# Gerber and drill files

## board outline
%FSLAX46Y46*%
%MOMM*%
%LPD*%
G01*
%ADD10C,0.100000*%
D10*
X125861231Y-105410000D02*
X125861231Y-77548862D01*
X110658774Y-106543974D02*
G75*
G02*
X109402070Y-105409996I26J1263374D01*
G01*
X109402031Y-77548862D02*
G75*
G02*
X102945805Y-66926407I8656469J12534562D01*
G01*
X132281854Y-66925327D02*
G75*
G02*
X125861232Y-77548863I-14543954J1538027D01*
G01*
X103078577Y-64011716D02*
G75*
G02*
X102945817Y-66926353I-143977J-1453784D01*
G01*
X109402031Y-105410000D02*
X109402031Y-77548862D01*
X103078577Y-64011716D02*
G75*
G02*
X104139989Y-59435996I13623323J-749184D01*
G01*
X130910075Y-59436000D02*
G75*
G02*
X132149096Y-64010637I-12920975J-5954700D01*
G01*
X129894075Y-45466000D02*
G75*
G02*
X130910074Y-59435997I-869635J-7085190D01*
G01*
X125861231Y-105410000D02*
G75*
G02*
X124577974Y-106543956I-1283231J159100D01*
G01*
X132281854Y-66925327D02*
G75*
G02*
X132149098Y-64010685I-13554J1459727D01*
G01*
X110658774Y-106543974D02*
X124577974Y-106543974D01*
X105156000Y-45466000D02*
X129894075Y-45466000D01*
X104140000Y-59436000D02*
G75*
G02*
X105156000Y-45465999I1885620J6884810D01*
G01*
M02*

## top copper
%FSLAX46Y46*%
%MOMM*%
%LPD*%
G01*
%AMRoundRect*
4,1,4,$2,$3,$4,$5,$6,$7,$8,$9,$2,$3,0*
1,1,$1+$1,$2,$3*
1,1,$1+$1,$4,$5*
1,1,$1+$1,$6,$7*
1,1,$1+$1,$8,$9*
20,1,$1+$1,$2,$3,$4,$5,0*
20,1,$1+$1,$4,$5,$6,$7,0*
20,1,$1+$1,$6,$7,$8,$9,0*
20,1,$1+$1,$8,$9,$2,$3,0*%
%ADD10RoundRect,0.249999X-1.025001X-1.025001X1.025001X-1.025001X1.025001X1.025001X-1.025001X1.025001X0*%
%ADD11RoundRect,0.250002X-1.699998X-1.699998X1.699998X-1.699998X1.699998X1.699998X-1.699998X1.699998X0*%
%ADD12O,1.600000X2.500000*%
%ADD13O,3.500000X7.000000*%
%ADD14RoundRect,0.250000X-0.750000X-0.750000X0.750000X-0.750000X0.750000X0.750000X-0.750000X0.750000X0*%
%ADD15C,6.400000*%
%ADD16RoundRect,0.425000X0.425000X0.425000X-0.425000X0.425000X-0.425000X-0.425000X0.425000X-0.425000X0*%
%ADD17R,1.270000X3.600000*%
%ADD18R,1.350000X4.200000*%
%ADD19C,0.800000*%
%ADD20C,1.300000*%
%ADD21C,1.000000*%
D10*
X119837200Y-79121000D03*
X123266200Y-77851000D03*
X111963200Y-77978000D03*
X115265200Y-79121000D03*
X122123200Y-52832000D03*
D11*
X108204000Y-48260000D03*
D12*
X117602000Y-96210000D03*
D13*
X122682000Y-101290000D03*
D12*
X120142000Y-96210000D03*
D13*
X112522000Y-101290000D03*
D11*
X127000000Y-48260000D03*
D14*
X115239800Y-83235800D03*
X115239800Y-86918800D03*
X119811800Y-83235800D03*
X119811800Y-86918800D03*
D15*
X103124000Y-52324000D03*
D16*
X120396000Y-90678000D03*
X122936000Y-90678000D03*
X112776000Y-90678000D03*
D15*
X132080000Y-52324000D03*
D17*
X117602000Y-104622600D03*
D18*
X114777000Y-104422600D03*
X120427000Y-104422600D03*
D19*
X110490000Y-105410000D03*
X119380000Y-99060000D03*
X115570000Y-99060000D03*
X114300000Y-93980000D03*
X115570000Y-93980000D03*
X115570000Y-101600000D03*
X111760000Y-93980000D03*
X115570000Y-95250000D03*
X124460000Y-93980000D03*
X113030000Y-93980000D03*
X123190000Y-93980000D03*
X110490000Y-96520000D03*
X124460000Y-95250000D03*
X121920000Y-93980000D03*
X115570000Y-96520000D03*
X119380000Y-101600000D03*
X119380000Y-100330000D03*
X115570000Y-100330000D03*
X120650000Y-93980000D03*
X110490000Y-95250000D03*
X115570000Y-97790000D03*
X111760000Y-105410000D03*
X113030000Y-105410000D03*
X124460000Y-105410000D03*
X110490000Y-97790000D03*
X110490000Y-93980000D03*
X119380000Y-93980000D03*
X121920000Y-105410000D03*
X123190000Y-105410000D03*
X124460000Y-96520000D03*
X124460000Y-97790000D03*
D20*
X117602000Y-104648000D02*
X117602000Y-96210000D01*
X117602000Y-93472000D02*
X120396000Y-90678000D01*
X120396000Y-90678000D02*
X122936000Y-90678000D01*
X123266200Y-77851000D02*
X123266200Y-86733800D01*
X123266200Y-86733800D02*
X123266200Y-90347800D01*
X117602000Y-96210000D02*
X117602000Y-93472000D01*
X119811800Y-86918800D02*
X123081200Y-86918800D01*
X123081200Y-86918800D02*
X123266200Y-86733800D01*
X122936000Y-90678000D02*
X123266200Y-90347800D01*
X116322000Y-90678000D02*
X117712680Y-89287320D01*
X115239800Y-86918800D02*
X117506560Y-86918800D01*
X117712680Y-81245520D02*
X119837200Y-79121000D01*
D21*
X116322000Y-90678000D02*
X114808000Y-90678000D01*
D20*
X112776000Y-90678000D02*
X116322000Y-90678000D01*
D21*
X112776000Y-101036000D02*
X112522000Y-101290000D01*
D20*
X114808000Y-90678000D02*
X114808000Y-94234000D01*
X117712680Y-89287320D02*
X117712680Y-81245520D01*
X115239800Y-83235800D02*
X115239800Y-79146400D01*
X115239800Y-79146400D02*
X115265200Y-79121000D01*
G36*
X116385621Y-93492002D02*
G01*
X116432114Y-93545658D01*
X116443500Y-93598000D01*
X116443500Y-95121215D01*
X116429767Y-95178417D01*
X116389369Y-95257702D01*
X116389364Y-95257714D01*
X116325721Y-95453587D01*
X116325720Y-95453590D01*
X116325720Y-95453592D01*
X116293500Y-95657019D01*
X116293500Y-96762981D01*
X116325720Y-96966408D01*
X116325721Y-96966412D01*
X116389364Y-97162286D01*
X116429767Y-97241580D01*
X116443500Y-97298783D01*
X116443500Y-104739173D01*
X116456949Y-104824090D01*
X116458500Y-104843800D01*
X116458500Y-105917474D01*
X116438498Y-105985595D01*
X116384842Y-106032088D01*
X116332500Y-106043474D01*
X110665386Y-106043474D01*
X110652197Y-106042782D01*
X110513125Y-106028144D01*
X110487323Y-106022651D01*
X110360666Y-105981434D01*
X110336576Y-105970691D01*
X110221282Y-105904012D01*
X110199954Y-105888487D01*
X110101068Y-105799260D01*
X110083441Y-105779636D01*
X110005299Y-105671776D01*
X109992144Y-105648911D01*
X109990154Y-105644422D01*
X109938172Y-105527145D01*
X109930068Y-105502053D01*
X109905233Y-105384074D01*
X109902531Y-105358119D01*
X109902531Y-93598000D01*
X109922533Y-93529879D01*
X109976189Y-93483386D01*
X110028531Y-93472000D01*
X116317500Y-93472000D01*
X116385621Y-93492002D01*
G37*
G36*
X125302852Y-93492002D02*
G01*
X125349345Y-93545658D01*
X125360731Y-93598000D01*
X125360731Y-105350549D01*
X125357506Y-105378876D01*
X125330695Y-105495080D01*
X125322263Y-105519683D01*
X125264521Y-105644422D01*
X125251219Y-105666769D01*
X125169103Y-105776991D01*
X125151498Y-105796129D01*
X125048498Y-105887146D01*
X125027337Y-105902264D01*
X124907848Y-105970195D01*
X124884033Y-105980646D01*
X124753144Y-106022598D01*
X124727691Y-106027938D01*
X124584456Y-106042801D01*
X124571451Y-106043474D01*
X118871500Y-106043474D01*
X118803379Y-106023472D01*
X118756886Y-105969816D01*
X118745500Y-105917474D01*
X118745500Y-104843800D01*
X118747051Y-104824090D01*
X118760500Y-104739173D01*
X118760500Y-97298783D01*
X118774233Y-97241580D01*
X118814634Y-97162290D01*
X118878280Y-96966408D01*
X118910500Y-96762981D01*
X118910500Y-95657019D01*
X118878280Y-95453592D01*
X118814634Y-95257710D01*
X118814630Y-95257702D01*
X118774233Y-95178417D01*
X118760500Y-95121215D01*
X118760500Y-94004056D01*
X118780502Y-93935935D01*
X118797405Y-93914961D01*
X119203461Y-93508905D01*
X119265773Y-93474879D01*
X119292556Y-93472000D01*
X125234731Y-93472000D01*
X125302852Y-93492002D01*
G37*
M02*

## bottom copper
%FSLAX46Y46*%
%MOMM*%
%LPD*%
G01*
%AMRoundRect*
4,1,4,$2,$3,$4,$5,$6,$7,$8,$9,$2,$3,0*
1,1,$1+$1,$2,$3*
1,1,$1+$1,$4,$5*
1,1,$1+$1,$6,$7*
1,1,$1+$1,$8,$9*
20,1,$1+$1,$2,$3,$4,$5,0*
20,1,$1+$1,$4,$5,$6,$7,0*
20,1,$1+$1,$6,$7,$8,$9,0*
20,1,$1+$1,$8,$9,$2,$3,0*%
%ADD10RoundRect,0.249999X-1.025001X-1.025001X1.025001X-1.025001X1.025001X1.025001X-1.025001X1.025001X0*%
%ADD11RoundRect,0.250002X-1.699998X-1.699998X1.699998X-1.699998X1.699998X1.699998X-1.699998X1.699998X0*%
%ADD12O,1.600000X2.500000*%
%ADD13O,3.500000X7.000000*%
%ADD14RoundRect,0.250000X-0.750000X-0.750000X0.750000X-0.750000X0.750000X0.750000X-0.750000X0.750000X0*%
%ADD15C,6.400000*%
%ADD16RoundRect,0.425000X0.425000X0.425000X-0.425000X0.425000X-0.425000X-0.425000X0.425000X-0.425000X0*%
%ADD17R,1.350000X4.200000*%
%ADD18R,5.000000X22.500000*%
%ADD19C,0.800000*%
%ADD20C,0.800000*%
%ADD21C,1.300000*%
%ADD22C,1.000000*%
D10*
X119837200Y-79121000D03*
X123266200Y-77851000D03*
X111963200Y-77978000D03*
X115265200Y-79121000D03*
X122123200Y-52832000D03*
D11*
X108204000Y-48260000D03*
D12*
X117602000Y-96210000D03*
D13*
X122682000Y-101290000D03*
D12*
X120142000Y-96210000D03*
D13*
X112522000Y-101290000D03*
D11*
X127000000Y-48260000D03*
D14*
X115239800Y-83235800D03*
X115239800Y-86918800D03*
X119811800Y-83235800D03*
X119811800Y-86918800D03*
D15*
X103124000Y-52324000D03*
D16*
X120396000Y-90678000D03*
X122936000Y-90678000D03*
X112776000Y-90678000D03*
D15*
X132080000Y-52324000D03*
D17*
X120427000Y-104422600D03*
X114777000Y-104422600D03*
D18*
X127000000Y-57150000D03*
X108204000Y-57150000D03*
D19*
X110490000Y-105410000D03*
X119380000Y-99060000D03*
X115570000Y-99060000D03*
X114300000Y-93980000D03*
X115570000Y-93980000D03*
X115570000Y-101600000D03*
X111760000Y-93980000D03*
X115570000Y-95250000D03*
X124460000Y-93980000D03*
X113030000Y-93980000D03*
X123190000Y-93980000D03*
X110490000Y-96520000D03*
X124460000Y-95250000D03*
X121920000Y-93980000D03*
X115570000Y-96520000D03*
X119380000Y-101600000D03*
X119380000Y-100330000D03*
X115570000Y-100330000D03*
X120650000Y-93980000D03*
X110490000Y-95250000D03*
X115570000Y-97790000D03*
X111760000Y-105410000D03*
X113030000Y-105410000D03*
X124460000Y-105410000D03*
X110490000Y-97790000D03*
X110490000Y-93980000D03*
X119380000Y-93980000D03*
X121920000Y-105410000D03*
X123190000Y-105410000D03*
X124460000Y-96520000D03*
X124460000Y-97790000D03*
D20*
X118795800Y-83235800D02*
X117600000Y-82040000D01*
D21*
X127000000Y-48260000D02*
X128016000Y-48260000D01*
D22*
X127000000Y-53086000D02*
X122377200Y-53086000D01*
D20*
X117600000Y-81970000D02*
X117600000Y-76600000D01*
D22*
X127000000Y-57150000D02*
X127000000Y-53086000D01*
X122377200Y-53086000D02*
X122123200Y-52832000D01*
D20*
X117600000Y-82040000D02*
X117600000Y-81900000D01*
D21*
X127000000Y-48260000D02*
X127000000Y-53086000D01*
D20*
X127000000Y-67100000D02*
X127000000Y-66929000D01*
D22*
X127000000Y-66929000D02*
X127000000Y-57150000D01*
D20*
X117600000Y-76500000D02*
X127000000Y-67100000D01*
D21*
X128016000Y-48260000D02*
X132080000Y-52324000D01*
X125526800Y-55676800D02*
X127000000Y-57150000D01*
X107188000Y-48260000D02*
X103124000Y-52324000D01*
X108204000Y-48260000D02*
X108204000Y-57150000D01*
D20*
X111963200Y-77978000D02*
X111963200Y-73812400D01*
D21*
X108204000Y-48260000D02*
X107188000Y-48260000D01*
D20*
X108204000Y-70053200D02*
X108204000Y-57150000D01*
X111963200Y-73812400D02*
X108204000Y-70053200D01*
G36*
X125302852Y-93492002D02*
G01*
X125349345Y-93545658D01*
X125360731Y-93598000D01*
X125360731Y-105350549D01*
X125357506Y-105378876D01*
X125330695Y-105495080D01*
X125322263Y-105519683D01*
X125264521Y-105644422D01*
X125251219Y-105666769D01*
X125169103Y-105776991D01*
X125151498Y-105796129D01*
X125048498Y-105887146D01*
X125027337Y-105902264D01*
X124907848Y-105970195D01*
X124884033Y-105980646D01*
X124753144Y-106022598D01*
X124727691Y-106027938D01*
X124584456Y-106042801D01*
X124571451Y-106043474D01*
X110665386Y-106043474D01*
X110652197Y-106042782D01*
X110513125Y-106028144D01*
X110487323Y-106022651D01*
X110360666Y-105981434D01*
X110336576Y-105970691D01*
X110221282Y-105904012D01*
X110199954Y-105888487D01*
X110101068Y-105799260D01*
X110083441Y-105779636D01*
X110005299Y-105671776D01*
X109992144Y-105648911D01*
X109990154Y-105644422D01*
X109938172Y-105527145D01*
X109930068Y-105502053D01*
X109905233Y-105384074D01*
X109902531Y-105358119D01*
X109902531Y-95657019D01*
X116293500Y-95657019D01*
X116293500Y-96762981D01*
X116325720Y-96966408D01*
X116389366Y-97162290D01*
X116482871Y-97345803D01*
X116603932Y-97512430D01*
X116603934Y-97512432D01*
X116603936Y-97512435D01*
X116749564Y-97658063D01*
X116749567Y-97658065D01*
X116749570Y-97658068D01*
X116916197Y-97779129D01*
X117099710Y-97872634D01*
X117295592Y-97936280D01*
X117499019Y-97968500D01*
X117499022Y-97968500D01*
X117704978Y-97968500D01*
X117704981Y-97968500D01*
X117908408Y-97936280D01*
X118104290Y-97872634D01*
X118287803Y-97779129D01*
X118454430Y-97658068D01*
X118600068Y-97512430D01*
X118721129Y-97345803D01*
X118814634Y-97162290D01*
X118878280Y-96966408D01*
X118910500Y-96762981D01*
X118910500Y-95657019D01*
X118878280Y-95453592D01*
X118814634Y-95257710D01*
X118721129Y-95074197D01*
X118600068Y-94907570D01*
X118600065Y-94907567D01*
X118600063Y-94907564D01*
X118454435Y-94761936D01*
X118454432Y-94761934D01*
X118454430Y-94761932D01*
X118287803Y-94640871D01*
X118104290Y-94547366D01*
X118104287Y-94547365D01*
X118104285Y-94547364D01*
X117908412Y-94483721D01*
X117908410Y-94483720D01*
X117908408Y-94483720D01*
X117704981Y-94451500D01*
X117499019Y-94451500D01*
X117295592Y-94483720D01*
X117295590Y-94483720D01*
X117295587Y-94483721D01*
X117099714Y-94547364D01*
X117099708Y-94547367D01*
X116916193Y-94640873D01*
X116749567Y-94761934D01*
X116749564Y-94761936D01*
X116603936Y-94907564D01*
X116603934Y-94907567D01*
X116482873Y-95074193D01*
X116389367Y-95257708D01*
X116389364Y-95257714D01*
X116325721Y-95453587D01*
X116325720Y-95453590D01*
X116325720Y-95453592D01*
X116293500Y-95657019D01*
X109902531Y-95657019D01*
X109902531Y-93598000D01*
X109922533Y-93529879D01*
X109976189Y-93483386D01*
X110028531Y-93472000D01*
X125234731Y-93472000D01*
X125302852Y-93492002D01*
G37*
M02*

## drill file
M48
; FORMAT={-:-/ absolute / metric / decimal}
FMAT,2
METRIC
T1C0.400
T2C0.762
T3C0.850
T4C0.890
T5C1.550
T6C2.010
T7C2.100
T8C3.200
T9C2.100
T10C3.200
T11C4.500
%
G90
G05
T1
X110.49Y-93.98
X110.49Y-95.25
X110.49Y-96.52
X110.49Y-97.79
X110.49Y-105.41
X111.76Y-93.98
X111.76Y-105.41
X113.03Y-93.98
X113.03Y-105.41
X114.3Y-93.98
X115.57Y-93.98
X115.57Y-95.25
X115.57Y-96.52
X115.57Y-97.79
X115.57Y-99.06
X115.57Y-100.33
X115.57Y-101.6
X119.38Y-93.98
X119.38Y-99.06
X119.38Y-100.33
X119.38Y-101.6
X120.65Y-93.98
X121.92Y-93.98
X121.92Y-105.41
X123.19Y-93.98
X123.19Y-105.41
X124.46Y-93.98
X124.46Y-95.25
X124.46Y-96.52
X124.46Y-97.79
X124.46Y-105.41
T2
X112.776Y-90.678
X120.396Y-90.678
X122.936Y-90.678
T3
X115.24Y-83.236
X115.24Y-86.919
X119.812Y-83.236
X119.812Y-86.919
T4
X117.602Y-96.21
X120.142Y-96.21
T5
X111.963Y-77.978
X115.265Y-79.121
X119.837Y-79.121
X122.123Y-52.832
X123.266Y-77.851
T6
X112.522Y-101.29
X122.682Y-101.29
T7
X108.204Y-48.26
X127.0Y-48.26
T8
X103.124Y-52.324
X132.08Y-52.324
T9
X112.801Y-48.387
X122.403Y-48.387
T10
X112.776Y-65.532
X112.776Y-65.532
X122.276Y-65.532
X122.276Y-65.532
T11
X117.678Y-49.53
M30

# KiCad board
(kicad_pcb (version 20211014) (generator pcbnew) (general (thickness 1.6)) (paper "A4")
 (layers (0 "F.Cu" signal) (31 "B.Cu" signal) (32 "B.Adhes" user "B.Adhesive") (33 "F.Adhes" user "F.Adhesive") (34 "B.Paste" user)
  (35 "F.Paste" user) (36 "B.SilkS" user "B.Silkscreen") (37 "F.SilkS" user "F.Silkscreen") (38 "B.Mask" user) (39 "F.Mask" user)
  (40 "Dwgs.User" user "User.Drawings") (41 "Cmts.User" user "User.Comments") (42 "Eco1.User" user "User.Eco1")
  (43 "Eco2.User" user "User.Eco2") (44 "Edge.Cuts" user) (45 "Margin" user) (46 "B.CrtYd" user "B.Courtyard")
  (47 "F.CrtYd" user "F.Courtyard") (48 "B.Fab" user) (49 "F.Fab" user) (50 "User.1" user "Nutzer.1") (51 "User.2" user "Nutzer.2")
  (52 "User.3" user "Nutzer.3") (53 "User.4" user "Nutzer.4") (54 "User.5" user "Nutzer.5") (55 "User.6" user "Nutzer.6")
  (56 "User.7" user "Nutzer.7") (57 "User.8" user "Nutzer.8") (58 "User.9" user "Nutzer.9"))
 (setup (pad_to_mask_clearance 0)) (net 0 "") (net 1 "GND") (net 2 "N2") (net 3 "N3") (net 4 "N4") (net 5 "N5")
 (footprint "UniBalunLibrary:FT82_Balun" (layer "F.Cu") (at 117.602 65.532)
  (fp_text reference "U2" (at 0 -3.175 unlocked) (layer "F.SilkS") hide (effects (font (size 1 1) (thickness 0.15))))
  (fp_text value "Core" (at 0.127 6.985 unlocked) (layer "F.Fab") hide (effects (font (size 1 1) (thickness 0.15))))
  (pad "" np_thru_hole circle (at 4.6736 0) (size 3.2 3.2) (drill 3.2) (layers *.Cu *.Mask))
  (pad "" np_thru_hole circle (at -4.826 0) (size 3.2 3.2) (drill 3.2) (layers *.Cu *.Mask))
  (pad "" np_thru_hole circle (at -4.826 0) (size 3.2 3.2) (drill 3.2) (layers *.Cu *.Mask))
  (pad "" np_thru_hole circle (at 4.6736 0) (size 3.2 3.2) (drill 3.2) (layers *.Cu *.Mask))
  (pad "1" thru_hole roundrect (at 2.2352 13.589) (size 2.55 2.55) (drill 1.55) (layers *.Cu *.Mask) (roundrect_rratio 0.098039)
   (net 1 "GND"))
  (pad "2" thru_hole roundrect (at 5.6642 12.319) (size 2.55 2.55) (drill 1.55) (layers *.Cu *.Mask) (roundrect_rratio 0.098039)
   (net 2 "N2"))
  (pad "3" thru_hole roundrect (at -5.6388 12.446) (size 2.55 2.55) (drill 1.55) (layers *.Cu *.Mask) (roundrect_rratio 0.098039)
   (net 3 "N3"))
  (pad "4" thru_hole roundrect (at -2.3368 13.589) (size 2.55 2.55) (drill 1.55) (layers *.Cu *.Mask) (roundrect_rratio 0.098039)
   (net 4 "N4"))
  (pad "5" thru_hole roundrect (at 4.5212 -12.7) (size 2.55 2.55) (drill 1.55) (layers *.Cu *.Mask) (roundrect_rratio 0.098039) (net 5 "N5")))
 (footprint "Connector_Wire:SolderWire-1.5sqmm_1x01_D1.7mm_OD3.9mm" (layer "F.Cu") (at 108.204 48.26)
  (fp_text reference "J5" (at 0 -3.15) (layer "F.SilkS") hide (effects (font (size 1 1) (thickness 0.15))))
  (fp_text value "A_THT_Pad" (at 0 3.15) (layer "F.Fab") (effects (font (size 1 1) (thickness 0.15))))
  (pad "1" thru_hole roundrect (at 0 0) (size 3.9 3.9) (drill 2.1) (layers *.Cu *.Mask) (roundrect_rratio 0.064103) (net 3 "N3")))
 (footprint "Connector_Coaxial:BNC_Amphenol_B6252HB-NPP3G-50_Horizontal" (layer "F.Cu") (at 117.602 96.21 180)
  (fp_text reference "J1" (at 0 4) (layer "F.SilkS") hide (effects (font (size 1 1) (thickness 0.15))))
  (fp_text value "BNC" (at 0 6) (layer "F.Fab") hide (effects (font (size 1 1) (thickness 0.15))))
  (pad "1" thru_hole oval (at 0 0 180) (size 1.6 2.5) (drill 0.89) (layers *.Cu *.Mask) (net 2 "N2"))
  (pad "2" thru_hole oval (at -5.08 -5.08 180) (size 3.5 7) (drill 2.01) (layers *.Cu *.Mask) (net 1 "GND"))
  (pad "2" thru_hole oval (at -2.54 0 180) (size 1.6 2.5) (drill 0.89) (layers *.Cu *.Mask) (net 1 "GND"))
  (pad "2" thru_hole oval (at 5.08 -5.08 180) (size 3.5 7) (drill 2.01) (layers *.Cu *.Mask) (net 1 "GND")))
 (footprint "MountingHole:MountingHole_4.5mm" (layer "F.Cu") (at 117.6782 49.53)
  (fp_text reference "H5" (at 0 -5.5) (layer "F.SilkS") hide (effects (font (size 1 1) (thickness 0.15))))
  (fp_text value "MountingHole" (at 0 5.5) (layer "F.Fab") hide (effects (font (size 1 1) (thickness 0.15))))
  (pad "" np_thru_hole circle (at 0 0) (size 4.5 4.5) (drill 4.5) (layers *.Cu *.Mask)))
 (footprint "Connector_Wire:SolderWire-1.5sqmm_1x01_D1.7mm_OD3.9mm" (layer "F.Cu") (at 127 48.26)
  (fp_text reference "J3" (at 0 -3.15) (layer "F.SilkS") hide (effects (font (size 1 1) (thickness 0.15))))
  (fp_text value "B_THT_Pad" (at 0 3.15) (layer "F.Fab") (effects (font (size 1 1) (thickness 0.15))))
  (pad "1" thru_hole roundrect (at 0 0) (size 3.9 3.9) (drill 2.1) (layers *.Cu *.Mask) (roundrect_rratio 0.064103) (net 5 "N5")))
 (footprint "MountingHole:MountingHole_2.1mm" (layer "F.Cu") (at 112.8014 48.387)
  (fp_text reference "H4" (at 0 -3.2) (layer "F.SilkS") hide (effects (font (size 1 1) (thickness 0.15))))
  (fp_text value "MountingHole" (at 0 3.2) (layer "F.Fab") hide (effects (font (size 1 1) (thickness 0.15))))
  (pad "" np_thru_hole circle (at 0 0) (size 2.1 2.1) (drill 2.1) (layers *.Cu *.Mask)))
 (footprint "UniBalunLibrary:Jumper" (layer "F.Cu") (at 117.602 85.09)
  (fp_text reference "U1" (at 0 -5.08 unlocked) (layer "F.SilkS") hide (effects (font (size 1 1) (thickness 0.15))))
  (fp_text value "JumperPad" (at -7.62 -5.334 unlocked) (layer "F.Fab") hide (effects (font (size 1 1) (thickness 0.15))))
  (pad "1" thru_hole roundrect (at -2.3622 -1.8542) (size 2 2) (drill 0.85) (layers *.Cu *.Mask) (roundrect_rratio 0.125) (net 4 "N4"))
  (pad "2" thru_hole roundrect (at -2.3622 1.8288) (size 2 2) (drill 0.85) (layers *.Cu *.Mask) (roundrect_rratio 0.125) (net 1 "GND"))
  (pad "3" thru_hole roundrect (at 2.2098 -1.8542) (size 2 2) (drill 0.85) (layers *.Cu *.Mask) (roundrect_rratio 0.125) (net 5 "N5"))
  (pad "4" thru_hole roundrect (at 2.2098 1.8288) (size 2 2) (drill 0.85) (layers *.Cu *.Mask) (roundrect_rratio 0.125) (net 2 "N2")))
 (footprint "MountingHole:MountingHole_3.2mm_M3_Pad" (layer "F.Cu") (at 103.124 52.324)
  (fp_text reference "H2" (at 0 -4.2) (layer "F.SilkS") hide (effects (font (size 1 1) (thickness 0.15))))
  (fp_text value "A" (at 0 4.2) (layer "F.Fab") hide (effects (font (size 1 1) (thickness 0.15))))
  (pad "1" thru_hole circle (at 0 0) (size 6.4 6.4) (drill 3.2) (layers *.Cu *.Mask) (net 3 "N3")))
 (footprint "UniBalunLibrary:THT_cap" (layer "F.Cu") (at 117.856 90.678 180)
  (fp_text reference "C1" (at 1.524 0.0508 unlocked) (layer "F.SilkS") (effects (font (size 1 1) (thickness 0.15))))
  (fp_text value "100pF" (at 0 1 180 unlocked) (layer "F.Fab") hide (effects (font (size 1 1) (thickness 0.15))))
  (pad "1" thru_hole roundrect (at -2.54 0 180) (size 1.7 1.7) (drill 0.762) (layers *.Cu *.Mask) (roundrect_rratio 0.25) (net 2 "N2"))
  (pad "1" thru_hole roundrect (at -5.08 0 180) (size 1.7 1.7) (drill 0.762) (layers *.Cu *.Mask) (roundrect_rratio 0.25) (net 2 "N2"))
  (pad "2" thru_hole roundrect (at 5.08 0 180) (size 1.7 1.7) (drill 0.762) (layers *.Cu *.Mask) (roundrect_rratio 0.25) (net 1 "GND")))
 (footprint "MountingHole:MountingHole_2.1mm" (layer "F.Cu") (at 122.4026 48.387)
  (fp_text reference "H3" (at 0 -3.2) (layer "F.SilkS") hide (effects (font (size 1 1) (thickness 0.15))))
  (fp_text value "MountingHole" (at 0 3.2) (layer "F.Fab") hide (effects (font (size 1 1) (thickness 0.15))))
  (pad "" np_thru_hole circle (at 0 0) (size 2.1 2.1) (drill 2.1) (layers *.Cu *.Mask)))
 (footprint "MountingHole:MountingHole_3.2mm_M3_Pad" (layer "F.Cu") (at 132.08 52.324)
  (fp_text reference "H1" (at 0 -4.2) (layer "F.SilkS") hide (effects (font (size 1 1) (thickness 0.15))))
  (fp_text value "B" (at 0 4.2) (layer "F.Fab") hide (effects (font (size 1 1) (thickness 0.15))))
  (pad "1" thru_hole circle (at 0 0) (size 6.4 6.4) (drill 3.2) (layers *.Cu *.Mask) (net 5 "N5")))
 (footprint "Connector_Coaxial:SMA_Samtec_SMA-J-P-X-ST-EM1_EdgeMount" (layer "F.Cu") (at 117.602 104.4226)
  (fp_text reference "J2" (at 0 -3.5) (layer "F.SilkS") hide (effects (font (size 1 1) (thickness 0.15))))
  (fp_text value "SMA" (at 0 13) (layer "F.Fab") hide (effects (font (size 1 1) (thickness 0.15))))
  (pad "1" smd rect (at 0 0.2) (size 1.27 3.6) (layers "F.Cu" "F.Paste" "F.Mask") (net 2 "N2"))
  (pad "2" smd rect (at 2.825 0) (size 1.35 4.2) (layers "B.Cu" "B.Paste" "B.Mask") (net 1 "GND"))
  (pad "2" smd rect (at -2.825 0) (size 1.35 4.2) (layers "B.Cu" "B.Paste" "B.Mask") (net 1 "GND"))
  (pad "2" smd rect (at -2.825 0) (size 1.35 4.2) (layers "F.Cu" "F.Paste" "F.Mask") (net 1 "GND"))
  (pad "2" smd rect (at 2.825 0) (size 1.35 4.2) (layers "F.Cu" "F.Paste" "F.Mask") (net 1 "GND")))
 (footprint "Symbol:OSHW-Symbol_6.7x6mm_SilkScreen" (layer "F.Cu") (at 117.5 68.2)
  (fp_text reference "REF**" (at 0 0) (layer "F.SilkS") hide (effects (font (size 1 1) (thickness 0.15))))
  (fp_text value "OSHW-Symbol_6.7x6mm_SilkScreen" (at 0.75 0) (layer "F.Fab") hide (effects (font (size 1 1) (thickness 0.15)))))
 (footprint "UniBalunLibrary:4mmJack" (layer "B.Cu") (at 127.254 56.896 90)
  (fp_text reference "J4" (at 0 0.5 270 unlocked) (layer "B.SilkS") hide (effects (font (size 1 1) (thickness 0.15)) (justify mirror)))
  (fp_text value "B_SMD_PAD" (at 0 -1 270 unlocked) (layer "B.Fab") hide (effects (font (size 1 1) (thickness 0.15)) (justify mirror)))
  (pad "1" smd rect (at -0.254 -0.254 90) (size 22.5 5) (layers "B.Cu" "B.Mask") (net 5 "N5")))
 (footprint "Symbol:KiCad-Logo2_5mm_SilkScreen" (layer "B.Cu") (at 117.729 58.547 180)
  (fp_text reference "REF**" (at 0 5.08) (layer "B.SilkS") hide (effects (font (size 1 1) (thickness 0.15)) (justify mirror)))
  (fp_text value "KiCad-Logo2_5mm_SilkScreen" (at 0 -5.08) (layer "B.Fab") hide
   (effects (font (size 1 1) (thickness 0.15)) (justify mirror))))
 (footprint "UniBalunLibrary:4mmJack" (layer "B.Cu") (at 108.458 56.896 90)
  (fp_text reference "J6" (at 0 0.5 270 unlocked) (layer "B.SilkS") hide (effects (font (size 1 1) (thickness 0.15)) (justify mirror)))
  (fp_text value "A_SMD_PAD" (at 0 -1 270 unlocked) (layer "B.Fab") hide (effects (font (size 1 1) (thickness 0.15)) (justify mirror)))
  (pad "1" smd rect (at -0.254 -0.254 90) (size 22.5 5) (layers "B.Cu" "B.Mask") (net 3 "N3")))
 (gr_line (start 125.861231 105.41) (end 125.861231 77.548862) (layer "Edge.Cuts") (width 0.1))
 (gr_arc (start 110.658774 106.543974) (mid 109.812413 106.218577) (end 109.402031 105.41) (layer "Edge.Cuts") (width 0.1))
 (gr_arc (start 109.402031 77.548862) (mid 105.04112 72.92614) (end 102.945817 66.926406) (layer "Edge.Cuts") (width 0.1))
 (gr_arc (start 132.281854 66.925327) (mid 130.254542 72.952072) (end 125.861231 77.548862) (layer "Edge.Cuts") (width 0.1))
 (gr_arc (start 103.078577 64.011716) (mid 104.394 65.532) (end 102.945817 66.926406) (layer "Edge.Cuts") (width 0.1))
 (gr_line (start 109.402031 105.41) (end 109.402031 77.548862) (layer "Edge.Cuts") (width 0.1))
 (gr_arc (start 103.078577 64.011716) (mid 103.410896 61.677837) (end 104.14 59.436) (layer "Edge.Cuts") (width 0.1))
 (gr_arc (start 130.910075 59.436) (mid 131.721418 61.671361) (end 132.149094 64.010637) (layer "Edge.Cuts") (width 0.1))
 (gr_arc (start 129.894075 45.466) (mid 136.144 52.033405) (end 130.910075 59.436) (layer "Edge.Cuts") (width 0.1))
 (gr_arc (start 125.861231 105.41) (mid 125.43422 106.219858) (end 124.577974 106.543974) (layer "Edge.Cuts") (width 0.1))
 (gr_arc (start 132.281854 66.925327) (mid 130.81 65.532) (end 132.149094 64.010637) (layer "Edge.Cuts") (width 0.1))
 (gr_line (start 110.658774 106.543974) (end 124.577974 106.543974) (layer "Edge.Cuts") (width 0.1))
 (gr_line (start 105.156 45.466) (end 129.894075 45.466) (layer "Edge.Cuts") (width 0.1))
 (gr_arc (start 104.14 59.436) (mid 98.906069 52.033405) (end 105.156 45.466) (layer "Edge.Cuts") (width 0.1))
 (segment (start 117.602 104.648) (end 117.602 96.21) (width 1.3) (layer "F.Cu") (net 2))
 (segment (start 117.602 93.472) (end 120.396 90.678) (width 1.3) (layer "F.Cu") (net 2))
 (segment (start 120.396 90.678) (end 122.936 90.678) (width 1.3) (layer "F.Cu") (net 2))
 (segment (start 123.2662 77.851) (end 123.2662 86.7338) (width 1.3) (layer "F.Cu") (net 2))
 (segment (start 123.2662 86.7338) (end 123.2662 90.3478) (width 1.3) (layer "F.Cu") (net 2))
 (segment (start 117.602 96.21) (end 117.602 93.472) (width 1.3) (layer "F.Cu") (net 2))
 (segment (start 119.8118 86.9188) (end 123.0812 86.9188) (width 1.3) (layer "F.Cu") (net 2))
 (segment (start 123.0812 86.9188) (end 123.2662 86.7338) (width 1.3) (layer "F.Cu") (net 2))
 (segment (start 122.936 90.678) (end 123.2662 90.3478) (width 1.3) (layer "F.Cu") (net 2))
 (segment (start 116.322 90.678) (end 117.71268 89.28732) (width 1.3) (layer "F.Cu") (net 1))
 (segment (start 115.2398 86.9188) (end 117.50656 86.9188) (width 1.3) (layer "F.Cu") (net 1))
 (segment (start 117.71268 81.24552) (end 119.8372 79.121) (width 1.3) (layer "F.Cu") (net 1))
 (segment (start 116.322 90.678) (end 114.808 90.678) (width 1) (layer "F.Cu") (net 1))
 (segment (start 112.776 90.678) (end 116.322 90.678) (width 1.3) (layer "F.Cu") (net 1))
 (segment (start 112.776 101.036) (end 112.522 101.29) (width 1) (layer "F.Cu") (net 1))
 (segment (start 114.808 90.678) (end 114.808 94.234) (width 1.3) (layer "F.Cu") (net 1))
 (segment (start 117.71268 89.28732) (end 117.71268 81.24552) (width 1.3) (layer "F.Cu") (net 1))
 (via (at 110.49 105.41) (size 0.8) (drill 0.4) (layers "F.Cu" "B.Cu") (free) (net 1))
 (via (at 119.38 99.06) (size 0.8) (drill 0.4) (layers "F.Cu" "B.Cu") (free) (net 1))
 (via (at 115.57 99.06) (size 0.8) (drill 0.4) (layers "F.Cu" "B.Cu") (free) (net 1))
 (via (at 114.3 93.98) (size 0.8) (drill 0.4) (layers "F.Cu" "B.Cu") (free) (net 1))
 (via (at 115.57 93.98) (size 0.8) (drill 0.4) (layers "F.Cu" "B.Cu") (free) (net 1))
 (via (at 115.57 101.6) (size 0.8) (drill 0.4) (layers "F.Cu" "B.Cu") (free) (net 1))
 (via (at 111.76 93.98) (size 0.8) (drill 0.4) (layers "F.Cu" "B.Cu") (free) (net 1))
 (via (at 115.57 95.25) (size 0.8) (drill 0.4) (layers "F.Cu" "B.Cu") (free) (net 1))
 (via (at 124.46 93.98) (size 0.8) (drill 0.4) (layers "F.Cu" "B.Cu") (free) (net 1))
 (via (at 113.03 93.98) (size 0.8) (drill 0.4) (layers "F.Cu" "B.Cu") (free) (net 1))
 (via (at 123.19 93.98) (size 0.8) (drill 0.4) (layers "F.Cu" "B.Cu") (free) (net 1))
 (via (at 110.49 96.52) (size 0.8) (drill 0.4) (layers "F.Cu" "B.Cu") (free) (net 1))
 (via (at 124.46 95.25) (size 0.8) (drill 0.4) (layers "F.Cu" "B.Cu") (free) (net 1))
 (via (at 121.92 93.98) (size 0.8) (drill 0.4) (layers "F.Cu" "B.Cu") (free) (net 1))
 (via (at 115.57 96.52) (size 0.8) (drill 0.4) (layers "F.Cu" "B.Cu") (free) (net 1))
 (via (at 119.38 101.6) (size 0.8) (drill 0.4) (layers "F.Cu" "B.Cu") (free) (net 1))
 (via (at 119.38 100.33) (size 0.8) (drill 0.4) (layers "F.Cu" "B.Cu") (free) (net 1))
 (via (at 115.57 100.33) (size 0.8) (drill 0.4) (layers "F.Cu" "B.Cu") (free) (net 1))
 (via (at 120.65 93.98) (size 0.8) (drill 0.4) (layers "F.Cu" "B.Cu") (free) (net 1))
 (via (at 110.49 95.25) (size 0.8) (drill 0.4) (layers "F.Cu" "B.Cu") (free) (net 1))
 (via (at 115.57 97.79) (size 0.8) (drill 0.4) (layers "F.Cu" "B.Cu") (free) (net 1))
 (via (at 111.76 105.41) (size 0.8) (drill 0.4) (layers "F.Cu" "B.Cu") (free) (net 1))
 (via (at 113.03 105.41) (size 0.8) (drill 0.4) (layers "F.Cu" "B.Cu") (free) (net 1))
 (via (at 124.46 105.41) (size 0.8) (drill 0.4) (layers "F.Cu" "B.Cu") (free) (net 1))
 (via (at 110.49 97.79) (size 0.8) (drill 0.4) (layers "F.Cu" "B.Cu") (free) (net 1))
 (via (at 110.49 93.98) (size 0.8) (drill 0.4) (layers "F.Cu" "B.Cu") (free) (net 1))
 (via (at 119.38 93.98) (size 0.8) (drill 0.4) (layers "F.Cu" "B.Cu") (free) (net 1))
 (via (at 121.92 105.41) (size 0.8) (drill 0.4) (layers "F.Cu" "B.Cu") (free) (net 1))
 (via (at 123.19 105.41) (size 0.8) (drill 0.4) (layers "F.Cu" "B.Cu") (free) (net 1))
 (via (at 124.46 96.52) (size 0.8) (drill 0.4) (layers "F.Cu" "B.Cu") (free) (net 1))
 (via (at 124.46 97.79) (size 0.8) (drill 0.4) (layers "F.Cu" "B.Cu") (free) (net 1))
 (segment (start 118.7958 83.2358) (end 117.6 82.04) (width 0.8) (layer "B.Cu") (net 5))
 (segment (start 127 48.26) (end 128.016 48.26) (width 1.3) (layer "B.Cu") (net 5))
 (segment (start 127 53.086) (end 122.3772 53.086) (width 1) (layer "B.Cu") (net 5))
 (segment (start 117.6 81.97) (end 117.6 76.6) (width 0.8) (layer "B.Cu") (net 5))
 (segment (start 127 57.15) (end 127 53.086) (width 1) (layer "B.Cu") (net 5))
 (segment (start 122.3772 53.086) (end 122.1232 52.832) (width 1) (layer "B.Cu") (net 5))
 (segment (start 117.6 82.04) (end 117.6 81.9) (width 0.8) (layer "B.Cu") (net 5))
 (segment (start 127 48.26) (end 127 53.086) (width 1.3) (layer "B.Cu") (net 5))
 (segment (start 127 67.1) (end 127 66.929) (width 0.8) (layer "B.Cu") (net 5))
 (segment (start 127 66.929) (end 127 57.15) (width 1) (layer "B.Cu") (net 5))
 (segment (start 117.6 76.5) (end 127 67.1) (width 0.8) (layer "B.Cu") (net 5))
 (segment (start 128.016 48.26) (end 132.08 52.324) (width 1.3) (layer "B.Cu") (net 5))
 (segment (start 125.5268 55.6768) (end 127 57.15) (width 1.3) (layer "B.Cu") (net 5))
 (segment (start 115.2398 83.2358) (end 115.2398 79.1464) (width 1.3) (layer "F.Cu") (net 4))
 (segment (start 115.2398 79.1464) (end 115.2652 79.121) (width 1.3) (layer "F.Cu") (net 4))
 (segment (start 107.188 48.26) (end 103.124 52.324) (width 1.3) (layer "B.Cu") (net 3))
 (segment (start 108.204 48.26) (end 108.204 57.15) (width 1.3) (layer "B.Cu") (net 3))
 (segment (start 111.9632 77.978) (end 111.9632 73.8124) (width 0.8) (layer "B.Cu") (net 3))
 (segment (start 108.204 48.26) (end 107.188 48.26) (width 1.3) (layer "B.Cu") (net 3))
 (segment (start 108.204 70.0532) (end 108.204 57.15) (width 0.8) (layer "B.Cu") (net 3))
 (segment (start 111.9632 73.8124) (end 108.204 70.0532) (width 0.8) (layer "B.Cu") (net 3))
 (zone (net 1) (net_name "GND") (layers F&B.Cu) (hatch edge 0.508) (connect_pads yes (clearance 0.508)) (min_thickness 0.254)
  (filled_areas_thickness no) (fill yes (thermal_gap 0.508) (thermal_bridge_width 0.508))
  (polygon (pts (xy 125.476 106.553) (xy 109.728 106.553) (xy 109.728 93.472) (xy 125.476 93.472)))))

